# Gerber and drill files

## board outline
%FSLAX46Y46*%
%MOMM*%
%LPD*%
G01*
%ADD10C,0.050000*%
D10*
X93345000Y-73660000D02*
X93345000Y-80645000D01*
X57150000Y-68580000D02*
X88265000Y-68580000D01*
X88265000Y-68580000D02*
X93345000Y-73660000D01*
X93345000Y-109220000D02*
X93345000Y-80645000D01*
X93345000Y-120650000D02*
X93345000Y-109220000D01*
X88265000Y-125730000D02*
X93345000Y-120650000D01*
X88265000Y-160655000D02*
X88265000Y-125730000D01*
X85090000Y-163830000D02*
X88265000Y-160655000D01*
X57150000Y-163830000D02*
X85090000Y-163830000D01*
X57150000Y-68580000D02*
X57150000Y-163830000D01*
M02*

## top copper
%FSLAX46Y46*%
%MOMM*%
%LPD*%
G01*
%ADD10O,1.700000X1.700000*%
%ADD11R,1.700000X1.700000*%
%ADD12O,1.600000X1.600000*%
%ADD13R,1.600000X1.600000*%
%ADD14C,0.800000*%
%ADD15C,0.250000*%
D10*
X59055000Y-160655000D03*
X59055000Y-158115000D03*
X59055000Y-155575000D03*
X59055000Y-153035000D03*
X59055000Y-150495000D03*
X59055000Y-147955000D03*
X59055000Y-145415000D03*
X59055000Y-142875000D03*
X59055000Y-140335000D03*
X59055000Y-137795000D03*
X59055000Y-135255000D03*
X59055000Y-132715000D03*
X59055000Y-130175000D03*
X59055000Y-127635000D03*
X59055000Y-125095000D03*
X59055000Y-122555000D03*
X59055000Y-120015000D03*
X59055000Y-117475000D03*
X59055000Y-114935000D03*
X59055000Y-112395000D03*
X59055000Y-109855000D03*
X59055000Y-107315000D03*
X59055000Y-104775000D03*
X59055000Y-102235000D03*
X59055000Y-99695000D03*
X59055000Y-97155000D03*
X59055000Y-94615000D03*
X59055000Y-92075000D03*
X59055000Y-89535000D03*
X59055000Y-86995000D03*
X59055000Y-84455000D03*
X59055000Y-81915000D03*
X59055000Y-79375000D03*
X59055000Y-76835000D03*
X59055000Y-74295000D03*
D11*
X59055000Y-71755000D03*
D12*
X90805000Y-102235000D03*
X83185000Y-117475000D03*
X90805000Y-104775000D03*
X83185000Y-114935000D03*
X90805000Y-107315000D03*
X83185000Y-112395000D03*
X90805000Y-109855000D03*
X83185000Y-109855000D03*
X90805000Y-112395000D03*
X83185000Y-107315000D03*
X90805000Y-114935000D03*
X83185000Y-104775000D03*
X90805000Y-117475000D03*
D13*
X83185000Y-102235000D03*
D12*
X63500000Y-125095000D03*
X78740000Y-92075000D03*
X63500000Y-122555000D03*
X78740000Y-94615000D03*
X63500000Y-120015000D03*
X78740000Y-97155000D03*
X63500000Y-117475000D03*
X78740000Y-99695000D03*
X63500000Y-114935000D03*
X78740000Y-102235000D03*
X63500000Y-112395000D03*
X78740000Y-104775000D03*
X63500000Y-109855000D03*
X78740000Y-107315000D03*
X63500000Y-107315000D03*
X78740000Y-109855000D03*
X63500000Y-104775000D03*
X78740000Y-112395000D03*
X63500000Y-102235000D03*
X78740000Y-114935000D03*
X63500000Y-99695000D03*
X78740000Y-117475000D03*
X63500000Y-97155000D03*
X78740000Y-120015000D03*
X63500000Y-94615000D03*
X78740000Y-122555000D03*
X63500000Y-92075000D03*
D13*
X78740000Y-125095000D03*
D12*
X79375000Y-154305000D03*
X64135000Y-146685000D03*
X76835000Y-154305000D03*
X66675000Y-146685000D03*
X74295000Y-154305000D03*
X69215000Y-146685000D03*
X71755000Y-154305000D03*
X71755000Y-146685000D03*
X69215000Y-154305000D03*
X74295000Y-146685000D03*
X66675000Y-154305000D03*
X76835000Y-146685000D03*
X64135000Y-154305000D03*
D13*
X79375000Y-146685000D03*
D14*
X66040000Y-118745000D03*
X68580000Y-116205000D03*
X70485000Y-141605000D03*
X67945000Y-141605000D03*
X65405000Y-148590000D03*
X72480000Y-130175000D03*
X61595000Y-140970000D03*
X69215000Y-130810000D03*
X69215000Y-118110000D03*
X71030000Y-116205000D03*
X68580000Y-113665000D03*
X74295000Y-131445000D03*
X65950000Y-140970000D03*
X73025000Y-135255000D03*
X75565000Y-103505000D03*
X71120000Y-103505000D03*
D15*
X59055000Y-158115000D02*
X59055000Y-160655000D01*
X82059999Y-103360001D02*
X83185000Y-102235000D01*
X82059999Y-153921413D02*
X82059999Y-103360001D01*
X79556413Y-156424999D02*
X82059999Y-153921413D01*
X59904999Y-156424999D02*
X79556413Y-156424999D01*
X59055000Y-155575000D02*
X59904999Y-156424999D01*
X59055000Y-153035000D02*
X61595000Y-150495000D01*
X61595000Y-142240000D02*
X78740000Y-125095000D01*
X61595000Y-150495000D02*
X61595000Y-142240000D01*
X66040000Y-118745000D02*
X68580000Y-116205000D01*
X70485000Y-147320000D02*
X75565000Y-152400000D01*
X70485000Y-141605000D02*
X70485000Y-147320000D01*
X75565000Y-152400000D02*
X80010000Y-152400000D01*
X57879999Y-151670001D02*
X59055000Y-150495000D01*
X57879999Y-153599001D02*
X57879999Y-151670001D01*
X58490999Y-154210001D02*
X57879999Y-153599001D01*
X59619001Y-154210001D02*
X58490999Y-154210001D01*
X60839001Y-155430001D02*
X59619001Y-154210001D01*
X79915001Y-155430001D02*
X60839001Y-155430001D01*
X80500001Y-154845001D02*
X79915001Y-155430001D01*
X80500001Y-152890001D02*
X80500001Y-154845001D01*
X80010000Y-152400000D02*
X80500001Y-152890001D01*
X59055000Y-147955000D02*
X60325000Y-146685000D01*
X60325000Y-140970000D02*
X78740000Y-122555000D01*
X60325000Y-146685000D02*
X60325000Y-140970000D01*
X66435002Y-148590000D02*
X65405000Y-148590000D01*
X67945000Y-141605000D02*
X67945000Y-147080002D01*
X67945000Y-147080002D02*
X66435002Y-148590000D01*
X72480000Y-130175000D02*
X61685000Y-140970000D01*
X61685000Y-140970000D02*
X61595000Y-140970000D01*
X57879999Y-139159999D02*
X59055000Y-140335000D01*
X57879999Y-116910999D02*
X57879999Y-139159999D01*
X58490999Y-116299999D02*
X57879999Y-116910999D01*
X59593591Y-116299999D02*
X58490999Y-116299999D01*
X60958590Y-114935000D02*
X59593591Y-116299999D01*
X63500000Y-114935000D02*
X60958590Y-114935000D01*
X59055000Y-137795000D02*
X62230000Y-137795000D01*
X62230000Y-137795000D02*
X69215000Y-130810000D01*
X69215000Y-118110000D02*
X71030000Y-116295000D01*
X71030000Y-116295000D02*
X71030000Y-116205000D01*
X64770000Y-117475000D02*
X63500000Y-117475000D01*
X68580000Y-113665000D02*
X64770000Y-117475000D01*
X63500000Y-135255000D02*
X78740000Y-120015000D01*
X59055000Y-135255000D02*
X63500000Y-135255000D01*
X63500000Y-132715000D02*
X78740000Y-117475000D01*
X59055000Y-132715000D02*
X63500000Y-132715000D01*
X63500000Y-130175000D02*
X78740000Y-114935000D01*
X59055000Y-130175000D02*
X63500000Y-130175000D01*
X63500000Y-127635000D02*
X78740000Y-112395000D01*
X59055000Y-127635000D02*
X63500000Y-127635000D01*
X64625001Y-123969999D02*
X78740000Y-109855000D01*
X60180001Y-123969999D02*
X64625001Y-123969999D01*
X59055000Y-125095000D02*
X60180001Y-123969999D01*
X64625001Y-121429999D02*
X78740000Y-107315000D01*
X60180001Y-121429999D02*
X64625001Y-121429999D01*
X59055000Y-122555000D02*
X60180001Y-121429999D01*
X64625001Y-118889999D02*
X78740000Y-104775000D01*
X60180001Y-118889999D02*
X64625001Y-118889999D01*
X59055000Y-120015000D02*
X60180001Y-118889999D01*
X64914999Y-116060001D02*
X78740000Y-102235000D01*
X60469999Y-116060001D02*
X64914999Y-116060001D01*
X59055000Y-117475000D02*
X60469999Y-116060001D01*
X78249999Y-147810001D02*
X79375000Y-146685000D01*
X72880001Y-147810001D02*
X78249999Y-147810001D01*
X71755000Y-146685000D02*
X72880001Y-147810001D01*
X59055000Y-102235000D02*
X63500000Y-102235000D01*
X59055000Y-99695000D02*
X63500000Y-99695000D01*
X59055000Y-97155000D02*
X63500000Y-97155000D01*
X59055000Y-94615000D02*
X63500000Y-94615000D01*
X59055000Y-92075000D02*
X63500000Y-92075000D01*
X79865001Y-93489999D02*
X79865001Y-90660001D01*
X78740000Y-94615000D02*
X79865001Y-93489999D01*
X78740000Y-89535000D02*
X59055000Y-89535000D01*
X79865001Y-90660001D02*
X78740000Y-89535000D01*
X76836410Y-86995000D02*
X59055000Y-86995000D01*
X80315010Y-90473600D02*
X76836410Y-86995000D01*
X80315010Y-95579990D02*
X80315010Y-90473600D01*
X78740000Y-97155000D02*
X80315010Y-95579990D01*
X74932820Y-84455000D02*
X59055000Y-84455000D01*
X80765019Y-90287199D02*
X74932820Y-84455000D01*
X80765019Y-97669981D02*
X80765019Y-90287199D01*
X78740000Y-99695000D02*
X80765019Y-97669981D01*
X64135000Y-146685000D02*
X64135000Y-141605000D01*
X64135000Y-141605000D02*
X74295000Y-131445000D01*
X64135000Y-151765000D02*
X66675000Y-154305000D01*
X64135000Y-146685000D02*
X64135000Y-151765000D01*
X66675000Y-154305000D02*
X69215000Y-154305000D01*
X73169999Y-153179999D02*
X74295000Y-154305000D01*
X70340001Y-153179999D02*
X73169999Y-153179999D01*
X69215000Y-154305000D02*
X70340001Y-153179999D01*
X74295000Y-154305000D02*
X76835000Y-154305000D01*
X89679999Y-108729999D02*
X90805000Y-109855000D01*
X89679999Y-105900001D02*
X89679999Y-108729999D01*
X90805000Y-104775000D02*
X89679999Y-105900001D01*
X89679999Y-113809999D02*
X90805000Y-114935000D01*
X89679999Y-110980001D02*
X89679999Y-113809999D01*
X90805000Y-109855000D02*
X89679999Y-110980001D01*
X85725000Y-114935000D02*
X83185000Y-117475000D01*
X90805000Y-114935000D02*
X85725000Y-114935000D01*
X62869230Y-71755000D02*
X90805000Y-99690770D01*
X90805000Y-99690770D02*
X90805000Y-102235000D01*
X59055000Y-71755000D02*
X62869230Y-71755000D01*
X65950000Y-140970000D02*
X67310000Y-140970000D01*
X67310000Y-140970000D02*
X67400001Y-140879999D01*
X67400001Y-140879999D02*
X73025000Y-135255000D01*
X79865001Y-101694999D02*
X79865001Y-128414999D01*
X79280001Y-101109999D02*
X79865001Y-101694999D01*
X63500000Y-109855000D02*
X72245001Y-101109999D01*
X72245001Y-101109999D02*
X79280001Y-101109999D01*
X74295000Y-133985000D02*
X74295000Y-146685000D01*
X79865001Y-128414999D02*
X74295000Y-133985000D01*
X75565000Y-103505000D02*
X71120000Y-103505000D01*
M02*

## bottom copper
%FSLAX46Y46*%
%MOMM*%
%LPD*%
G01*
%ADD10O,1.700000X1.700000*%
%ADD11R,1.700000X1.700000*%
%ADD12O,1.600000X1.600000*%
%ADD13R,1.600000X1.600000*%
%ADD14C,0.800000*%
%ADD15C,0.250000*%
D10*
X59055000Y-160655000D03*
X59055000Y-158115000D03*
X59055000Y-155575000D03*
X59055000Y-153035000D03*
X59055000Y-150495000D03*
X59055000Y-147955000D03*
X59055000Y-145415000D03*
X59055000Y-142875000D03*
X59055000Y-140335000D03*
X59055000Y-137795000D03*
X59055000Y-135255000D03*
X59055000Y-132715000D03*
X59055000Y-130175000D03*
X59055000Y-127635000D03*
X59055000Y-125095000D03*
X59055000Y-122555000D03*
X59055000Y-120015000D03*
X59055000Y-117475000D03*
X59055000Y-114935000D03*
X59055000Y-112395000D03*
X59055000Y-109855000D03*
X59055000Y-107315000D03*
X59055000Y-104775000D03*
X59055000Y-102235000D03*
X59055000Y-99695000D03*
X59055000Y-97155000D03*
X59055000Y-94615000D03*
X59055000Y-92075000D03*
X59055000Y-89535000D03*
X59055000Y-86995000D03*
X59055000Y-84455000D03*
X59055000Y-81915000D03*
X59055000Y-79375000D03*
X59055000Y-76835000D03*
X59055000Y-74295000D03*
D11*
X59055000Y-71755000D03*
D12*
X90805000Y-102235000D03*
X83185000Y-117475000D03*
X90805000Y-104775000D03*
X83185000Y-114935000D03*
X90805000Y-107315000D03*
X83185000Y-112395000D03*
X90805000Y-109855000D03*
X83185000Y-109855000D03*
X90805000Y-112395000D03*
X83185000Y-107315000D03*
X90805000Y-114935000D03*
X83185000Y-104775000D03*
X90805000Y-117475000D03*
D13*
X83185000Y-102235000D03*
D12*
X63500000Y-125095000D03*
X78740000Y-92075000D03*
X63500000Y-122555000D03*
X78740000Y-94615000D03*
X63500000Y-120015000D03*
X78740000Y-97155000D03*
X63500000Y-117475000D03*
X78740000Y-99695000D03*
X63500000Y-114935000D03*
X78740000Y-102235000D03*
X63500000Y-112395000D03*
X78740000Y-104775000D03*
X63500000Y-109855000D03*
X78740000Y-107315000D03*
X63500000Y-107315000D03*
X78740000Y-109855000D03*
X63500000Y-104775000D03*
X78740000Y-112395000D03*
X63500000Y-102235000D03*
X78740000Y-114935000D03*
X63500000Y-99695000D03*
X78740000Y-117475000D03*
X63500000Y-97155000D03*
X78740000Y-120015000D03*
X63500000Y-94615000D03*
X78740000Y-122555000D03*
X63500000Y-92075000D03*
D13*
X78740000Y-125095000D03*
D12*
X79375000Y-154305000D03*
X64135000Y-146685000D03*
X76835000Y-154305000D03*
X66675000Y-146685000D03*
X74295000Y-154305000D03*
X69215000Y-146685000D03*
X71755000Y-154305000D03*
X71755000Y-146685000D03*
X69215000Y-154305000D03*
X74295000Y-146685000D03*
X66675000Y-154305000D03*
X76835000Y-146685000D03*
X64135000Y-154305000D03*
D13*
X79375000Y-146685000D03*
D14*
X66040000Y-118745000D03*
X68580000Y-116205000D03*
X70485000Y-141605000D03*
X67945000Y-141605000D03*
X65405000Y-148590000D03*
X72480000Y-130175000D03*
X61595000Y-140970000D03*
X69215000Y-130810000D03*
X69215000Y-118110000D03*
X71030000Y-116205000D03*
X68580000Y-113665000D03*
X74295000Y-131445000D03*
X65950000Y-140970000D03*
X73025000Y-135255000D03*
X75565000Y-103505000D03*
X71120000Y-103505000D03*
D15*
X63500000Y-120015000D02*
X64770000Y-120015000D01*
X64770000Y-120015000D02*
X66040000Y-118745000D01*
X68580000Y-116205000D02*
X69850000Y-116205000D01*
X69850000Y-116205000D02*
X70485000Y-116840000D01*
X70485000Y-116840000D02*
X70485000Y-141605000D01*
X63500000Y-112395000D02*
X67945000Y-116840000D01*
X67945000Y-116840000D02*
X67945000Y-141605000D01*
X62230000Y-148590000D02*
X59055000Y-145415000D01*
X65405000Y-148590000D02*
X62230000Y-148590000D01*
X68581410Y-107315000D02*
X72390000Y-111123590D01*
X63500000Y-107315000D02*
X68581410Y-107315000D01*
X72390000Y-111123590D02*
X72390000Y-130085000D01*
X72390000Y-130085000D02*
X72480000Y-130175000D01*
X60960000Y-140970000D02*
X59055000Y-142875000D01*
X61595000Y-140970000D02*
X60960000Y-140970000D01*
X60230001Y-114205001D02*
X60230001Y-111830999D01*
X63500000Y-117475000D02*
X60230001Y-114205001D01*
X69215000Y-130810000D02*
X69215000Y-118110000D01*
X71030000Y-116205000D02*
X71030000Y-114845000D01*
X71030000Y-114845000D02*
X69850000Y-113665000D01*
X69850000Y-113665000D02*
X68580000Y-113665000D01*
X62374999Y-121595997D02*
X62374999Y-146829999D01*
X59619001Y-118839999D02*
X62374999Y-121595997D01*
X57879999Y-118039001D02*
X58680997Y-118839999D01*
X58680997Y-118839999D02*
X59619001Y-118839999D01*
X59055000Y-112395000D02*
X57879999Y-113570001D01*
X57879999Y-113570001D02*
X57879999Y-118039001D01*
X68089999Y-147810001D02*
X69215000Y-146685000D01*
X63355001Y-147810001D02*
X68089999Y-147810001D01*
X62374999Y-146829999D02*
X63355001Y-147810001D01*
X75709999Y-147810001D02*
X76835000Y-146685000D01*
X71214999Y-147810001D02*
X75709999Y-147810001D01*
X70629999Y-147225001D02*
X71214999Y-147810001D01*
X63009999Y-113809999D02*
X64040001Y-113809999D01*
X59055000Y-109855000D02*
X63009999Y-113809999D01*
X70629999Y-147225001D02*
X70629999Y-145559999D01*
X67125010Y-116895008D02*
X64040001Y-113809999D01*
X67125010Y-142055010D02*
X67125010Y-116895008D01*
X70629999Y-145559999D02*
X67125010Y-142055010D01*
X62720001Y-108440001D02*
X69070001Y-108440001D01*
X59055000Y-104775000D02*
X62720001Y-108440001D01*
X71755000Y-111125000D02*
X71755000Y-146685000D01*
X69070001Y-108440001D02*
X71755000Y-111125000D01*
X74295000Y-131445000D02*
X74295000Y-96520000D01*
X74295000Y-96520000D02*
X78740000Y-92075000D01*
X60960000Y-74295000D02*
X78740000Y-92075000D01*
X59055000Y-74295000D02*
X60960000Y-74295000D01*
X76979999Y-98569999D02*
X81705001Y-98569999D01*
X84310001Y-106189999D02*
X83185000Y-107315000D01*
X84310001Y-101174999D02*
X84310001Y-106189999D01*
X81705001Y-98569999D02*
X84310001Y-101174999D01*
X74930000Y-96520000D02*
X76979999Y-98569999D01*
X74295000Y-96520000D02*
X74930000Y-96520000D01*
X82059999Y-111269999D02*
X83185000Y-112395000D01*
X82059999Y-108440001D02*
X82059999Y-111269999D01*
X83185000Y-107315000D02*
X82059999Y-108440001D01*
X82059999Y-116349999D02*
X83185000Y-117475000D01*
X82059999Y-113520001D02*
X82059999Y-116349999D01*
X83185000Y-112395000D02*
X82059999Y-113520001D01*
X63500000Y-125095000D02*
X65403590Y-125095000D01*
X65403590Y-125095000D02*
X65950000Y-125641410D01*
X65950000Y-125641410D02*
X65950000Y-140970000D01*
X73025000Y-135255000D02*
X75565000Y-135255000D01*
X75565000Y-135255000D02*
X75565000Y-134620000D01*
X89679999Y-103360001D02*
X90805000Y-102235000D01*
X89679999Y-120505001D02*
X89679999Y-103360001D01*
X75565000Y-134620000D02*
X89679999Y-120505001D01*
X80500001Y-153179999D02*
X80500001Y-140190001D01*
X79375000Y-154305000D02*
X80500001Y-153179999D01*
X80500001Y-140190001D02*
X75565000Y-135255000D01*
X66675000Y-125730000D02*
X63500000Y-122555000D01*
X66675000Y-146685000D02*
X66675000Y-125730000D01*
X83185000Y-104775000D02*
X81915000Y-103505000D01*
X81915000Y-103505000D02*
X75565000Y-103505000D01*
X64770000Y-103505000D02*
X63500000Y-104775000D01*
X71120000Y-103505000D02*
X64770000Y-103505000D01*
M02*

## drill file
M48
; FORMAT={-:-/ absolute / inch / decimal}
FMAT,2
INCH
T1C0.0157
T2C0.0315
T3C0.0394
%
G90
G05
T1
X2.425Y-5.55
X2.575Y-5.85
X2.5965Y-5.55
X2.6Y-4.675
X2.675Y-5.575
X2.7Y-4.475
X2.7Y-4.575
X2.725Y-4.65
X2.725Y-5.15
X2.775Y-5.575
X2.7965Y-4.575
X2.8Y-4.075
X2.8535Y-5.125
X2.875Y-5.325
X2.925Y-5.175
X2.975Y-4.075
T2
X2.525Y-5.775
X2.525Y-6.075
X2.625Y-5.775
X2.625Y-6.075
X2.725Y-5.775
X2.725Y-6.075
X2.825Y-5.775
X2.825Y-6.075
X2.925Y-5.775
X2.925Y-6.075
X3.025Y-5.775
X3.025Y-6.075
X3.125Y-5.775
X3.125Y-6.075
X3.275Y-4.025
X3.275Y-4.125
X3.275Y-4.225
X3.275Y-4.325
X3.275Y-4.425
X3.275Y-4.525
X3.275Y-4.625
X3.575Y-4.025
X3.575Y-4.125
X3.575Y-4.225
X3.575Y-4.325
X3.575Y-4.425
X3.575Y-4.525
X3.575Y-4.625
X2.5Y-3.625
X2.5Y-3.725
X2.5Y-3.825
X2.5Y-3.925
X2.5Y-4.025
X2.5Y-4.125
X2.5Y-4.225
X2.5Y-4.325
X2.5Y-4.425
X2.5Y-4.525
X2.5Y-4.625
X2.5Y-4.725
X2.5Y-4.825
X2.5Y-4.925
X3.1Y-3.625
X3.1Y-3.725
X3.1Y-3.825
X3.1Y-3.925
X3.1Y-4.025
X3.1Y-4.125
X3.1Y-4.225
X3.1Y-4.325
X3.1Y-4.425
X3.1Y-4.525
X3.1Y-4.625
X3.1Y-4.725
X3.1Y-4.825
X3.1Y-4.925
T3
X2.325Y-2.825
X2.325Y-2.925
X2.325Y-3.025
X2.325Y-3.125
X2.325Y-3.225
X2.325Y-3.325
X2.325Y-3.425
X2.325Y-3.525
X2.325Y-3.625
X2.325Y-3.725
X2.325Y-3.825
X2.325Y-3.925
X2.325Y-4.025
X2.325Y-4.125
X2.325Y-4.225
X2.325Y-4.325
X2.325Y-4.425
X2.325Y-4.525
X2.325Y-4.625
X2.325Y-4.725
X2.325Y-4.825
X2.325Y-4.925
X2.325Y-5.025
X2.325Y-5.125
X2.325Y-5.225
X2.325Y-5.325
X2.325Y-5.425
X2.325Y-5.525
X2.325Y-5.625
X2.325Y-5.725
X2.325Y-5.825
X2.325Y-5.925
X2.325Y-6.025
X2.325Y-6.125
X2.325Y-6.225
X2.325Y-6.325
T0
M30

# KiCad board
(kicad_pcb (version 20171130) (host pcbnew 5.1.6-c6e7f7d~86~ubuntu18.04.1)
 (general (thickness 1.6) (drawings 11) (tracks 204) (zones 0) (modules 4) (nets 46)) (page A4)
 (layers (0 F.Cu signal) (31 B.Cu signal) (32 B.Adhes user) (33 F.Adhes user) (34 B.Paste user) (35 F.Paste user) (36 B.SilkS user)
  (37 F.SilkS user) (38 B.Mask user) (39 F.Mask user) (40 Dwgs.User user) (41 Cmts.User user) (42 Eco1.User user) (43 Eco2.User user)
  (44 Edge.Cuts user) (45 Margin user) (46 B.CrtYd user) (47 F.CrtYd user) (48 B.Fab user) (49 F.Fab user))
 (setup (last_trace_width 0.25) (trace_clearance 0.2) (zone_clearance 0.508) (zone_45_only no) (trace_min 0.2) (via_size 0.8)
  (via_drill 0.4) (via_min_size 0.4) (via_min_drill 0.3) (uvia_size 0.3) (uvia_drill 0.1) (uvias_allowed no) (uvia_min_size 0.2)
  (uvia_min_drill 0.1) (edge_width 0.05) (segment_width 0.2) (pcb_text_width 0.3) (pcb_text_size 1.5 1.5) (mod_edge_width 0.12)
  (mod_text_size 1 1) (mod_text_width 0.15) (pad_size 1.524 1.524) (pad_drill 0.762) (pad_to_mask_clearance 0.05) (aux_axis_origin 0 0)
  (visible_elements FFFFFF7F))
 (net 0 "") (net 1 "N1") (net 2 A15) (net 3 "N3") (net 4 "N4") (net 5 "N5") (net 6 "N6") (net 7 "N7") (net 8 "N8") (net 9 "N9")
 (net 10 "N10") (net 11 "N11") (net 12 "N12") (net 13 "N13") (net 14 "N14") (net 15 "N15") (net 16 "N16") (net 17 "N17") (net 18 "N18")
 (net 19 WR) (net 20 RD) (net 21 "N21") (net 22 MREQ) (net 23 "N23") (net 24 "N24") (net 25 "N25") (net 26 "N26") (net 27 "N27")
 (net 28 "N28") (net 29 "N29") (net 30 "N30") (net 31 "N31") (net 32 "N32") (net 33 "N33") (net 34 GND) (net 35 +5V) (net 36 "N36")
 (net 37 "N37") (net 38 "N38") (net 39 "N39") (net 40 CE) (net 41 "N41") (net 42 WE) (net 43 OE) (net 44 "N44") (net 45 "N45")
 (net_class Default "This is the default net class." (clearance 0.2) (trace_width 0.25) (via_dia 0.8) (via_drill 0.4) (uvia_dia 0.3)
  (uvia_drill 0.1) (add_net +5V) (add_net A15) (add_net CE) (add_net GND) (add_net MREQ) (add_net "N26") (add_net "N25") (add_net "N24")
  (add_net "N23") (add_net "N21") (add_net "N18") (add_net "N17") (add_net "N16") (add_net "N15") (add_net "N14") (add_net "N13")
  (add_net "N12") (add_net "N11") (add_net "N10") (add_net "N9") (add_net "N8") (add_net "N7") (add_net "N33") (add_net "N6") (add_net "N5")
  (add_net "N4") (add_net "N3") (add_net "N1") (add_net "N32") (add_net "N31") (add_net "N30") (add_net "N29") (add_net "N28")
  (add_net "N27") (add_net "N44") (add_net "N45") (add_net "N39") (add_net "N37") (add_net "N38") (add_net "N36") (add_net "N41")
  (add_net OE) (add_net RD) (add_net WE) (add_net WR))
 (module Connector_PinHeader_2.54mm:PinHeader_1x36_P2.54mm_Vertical (layer F.Cu) (at 59.055 71.755)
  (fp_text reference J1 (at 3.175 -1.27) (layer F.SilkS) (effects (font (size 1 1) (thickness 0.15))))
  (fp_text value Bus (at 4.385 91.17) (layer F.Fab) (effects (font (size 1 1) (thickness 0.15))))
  (pad 36 thru_hole oval (at 0 88.9) (size 1.7 1.7) (drill 1) (layers *.Cu *.Mask) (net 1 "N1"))
  (pad 35 thru_hole oval (at 0 86.36) (size 1.7 1.7) (drill 1) (layers *.Cu *.Mask) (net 1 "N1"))
  (pad 34 thru_hole oval (at 0 83.82) (size 1.7 1.7) (drill 1) (layers *.Cu *.Mask) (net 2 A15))
  (pad 33 thru_hole oval (at 0 81.28) (size 1.7 1.7) (drill 1) (layers *.Cu *.Mask) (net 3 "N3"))
  (pad 32 thru_hole oval (at 0 78.74) (size 1.7 1.7) (drill 1) (layers *.Cu *.Mask) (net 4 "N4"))
  (pad 31 thru_hole oval (at 0 76.2) (size 1.7 1.7) (drill 1) (layers *.Cu *.Mask) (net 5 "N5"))
  (pad 30 thru_hole oval (at 0 73.66) (size 1.7 1.7) (drill 1) (layers *.Cu *.Mask) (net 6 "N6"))
  (pad 29 thru_hole oval (at 0 71.12) (size 1.7 1.7) (drill 1) (layers *.Cu *.Mask) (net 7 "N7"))
  (pad 28 thru_hole oval (at 0 68.58) (size 1.7 1.7) (drill 1) (layers *.Cu *.Mask) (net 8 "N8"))
  (pad 27 thru_hole oval (at 0 66.04) (size 1.7 1.7) (drill 1) (layers *.Cu *.Mask) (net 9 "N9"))
  (pad 26 thru_hole oval (at 0 63.5) (size 1.7 1.7) (drill 1) (layers *.Cu *.Mask) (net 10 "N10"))
  (pad 25 thru_hole oval (at 0 60.96) (size 1.7 1.7) (drill 1) (layers *.Cu *.Mask) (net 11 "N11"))
  (pad 24 thru_hole oval (at 0 58.42) (size 1.7 1.7) (drill 1) (layers *.Cu *.Mask) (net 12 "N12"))
  (pad 23 thru_hole oval (at 0 55.88) (size 1.7 1.7) (drill 1) (layers *.Cu *.Mask) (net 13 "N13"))
  (pad 22 thru_hole oval (at 0 53.34) (size 1.7 1.7) (drill 1) (layers *.Cu *.Mask) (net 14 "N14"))
  (pad 21 thru_hole oval (at 0 50.8) (size 1.7 1.7) (drill 1) (layers *.Cu *.Mask) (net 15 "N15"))
  (pad 20 thru_hole oval (at 0 48.26) (size 1.7 1.7) (drill 1) (layers *.Cu *.Mask) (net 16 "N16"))
  (pad 19 thru_hole oval (at 0 45.72) (size 1.7 1.7) (drill 1) (layers *.Cu *.Mask) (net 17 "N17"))
  (pad 18 thru_hole oval (at 0 43.18) (size 1.7 1.7) (drill 1) (layers *.Cu *.Mask) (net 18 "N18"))
  (pad 17 thru_hole oval (at 0 40.64) (size 1.7 1.7) (drill 1) (layers *.Cu *.Mask) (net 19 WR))
  (pad 16 thru_hole oval (at 0 38.1) (size 1.7 1.7) (drill 1) (layers *.Cu *.Mask) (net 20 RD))
  (pad 15 thru_hole oval (at 0 35.56) (size 1.7 1.7) (drill 1) (layers *.Cu *.Mask) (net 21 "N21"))
  (pad 14 thru_hole oval (at 0 33.02) (size 1.7 1.7) (drill 1) (layers *.Cu *.Mask) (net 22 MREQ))
  (pad 13 thru_hole oval (at 0 30.48) (size 1.7 1.7) (drill 1) (layers *.Cu *.Mask) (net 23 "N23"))
  (pad 12 thru_hole oval (at 0 27.94) (size 1.7 1.7) (drill 1) (layers *.Cu *.Mask) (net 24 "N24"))
  (pad 11 thru_hole oval (at 0 25.4) (size 1.7 1.7) (drill 1) (layers *.Cu *.Mask) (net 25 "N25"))
  (pad 10 thru_hole oval (at 0 22.86) (size 1.7 1.7) (drill 1) (layers *.Cu *.Mask) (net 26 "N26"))
  (pad 9 thru_hole oval (at 0 20.32) (size 1.7 1.7) (drill 1) (layers *.Cu *.Mask) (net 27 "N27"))
  (pad 8 thru_hole oval (at 0 17.78) (size 1.7 1.7) (drill 1) (layers *.Cu *.Mask) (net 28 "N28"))
  (pad 7 thru_hole oval (at 0 15.24) (size 1.7 1.7) (drill 1) (layers *.Cu *.Mask) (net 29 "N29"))
  (pad 6 thru_hole oval (at 0 12.7) (size 1.7 1.7) (drill 1) (layers *.Cu *.Mask) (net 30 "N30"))
  (pad 5 thru_hole oval (at 0 10.16) (size 1.7 1.7) (drill 1) (layers *.Cu *.Mask) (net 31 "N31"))
  (pad 4 thru_hole oval (at 0 7.62) (size 1.7 1.7) (drill 1) (layers *.Cu *.Mask) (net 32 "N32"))
  (pad 3 thru_hole oval (at 0 5.08) (size 1.7 1.7) (drill 1) (layers *.Cu *.Mask) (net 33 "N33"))
  (pad 2 thru_hole oval (at 0 2.54) (size 1.7 1.7) (drill 1) (layers *.Cu *.Mask) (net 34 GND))
  (pad 1 thru_hole rect (at 0 0) (size 1.7 1.7) (drill 1) (layers *.Cu *.Mask) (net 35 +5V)))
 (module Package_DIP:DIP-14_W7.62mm (layer F.Cu) (at 83.185 102.235)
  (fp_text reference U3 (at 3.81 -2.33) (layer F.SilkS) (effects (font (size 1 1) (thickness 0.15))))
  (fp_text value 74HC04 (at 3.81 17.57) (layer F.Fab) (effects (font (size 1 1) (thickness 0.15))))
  (pad 14 thru_hole oval (at 7.62 0) (size 1.6 1.6) (drill 0.8) (layers *.Cu *.Mask) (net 35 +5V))
  (pad 7 thru_hole oval (at 0 15.24) (size 1.6 1.6) (drill 0.8) (layers *.Cu *.Mask) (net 34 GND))
  (pad 13 thru_hole oval (at 7.62 2.54) (size 1.6 1.6) (drill 0.8) (layers *.Cu *.Mask) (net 34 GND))
  (pad 6 thru_hole oval (at 0 12.7) (size 1.6 1.6) (drill 0.8) (layers *.Cu *.Mask) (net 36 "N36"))
  (pad 12 thru_hole oval (at 7.62 5.08) (size 1.6 1.6) (drill 0.8) (layers *.Cu *.Mask) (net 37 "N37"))
  (pad 5 thru_hole oval (at 0 10.16) (size 1.6 1.6) (drill 0.8) (layers *.Cu *.Mask) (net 34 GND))
  (pad 11 thru_hole oval (at 7.62 7.62) (size 1.6 1.6) (drill 0.8) (layers *.Cu *.Mask) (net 34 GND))
  (pad 4 thru_hole oval (at 0 7.62) (size 1.6 1.6) (drill 0.8) (layers *.Cu *.Mask) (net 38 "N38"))
  (pad 10 thru_hole oval (at 7.62 10.16) (size 1.6 1.6) (drill 0.8) (layers *.Cu *.Mask) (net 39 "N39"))
  (pad 3 thru_hole oval (at 0 5.08) (size 1.6 1.6) (drill 0.8) (layers *.Cu *.Mask) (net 34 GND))
  (pad 9 thru_hole oval (at 7.62 12.7) (size 1.6 1.6) (drill 0.8) (layers *.Cu *.Mask) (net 34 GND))
  (pad 2 thru_hole oval (at 0 2.54) (size 1.6 1.6) (drill 0.8) (layers *.Cu *.Mask) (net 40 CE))
  (pad 8 thru_hole oval (at 7.62 15.24) (size 1.6 1.6) (drill 0.8) (layers *.Cu *.Mask) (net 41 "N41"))
  (pad 1 thru_hole rect (at 0 0) (size 1.6 1.6) (drill 0.8) (layers *.Cu *.Mask) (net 2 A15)))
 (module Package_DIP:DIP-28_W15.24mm (layer F.Cu) (at 78.74 125.095 180)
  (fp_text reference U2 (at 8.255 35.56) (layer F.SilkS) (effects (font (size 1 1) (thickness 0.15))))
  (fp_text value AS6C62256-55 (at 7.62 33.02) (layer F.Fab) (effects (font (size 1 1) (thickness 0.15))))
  (pad 28 thru_hole oval (at 15.24 0 180) (size 1.6 1.6) (drill 0.8) (layers *.Cu *.Mask) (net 35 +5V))
  (pad 14 thru_hole oval (at 0 33.02 180) (size 1.6 1.6) (drill 0.8) (layers *.Cu *.Mask) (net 34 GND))
  (pad 27 thru_hole oval (at 15.24 2.54 180) (size 1.6 1.6) (drill 0.8) (layers *.Cu *.Mask) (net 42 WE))
  (pad 13 thru_hole oval (at 0 30.48 180) (size 1.6 1.6) (drill 0.8) (layers *.Cu *.Mask) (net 28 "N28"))
  (pad 26 thru_hole oval (at 15.24 5.08 180) (size 1.6 1.6) (drill 0.8) (layers *.Cu *.Mask) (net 4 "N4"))
  (pad 12 thru_hole oval (at 0 27.94 180) (size 1.6 1.6) (drill 0.8) (layers *.Cu *.Mask) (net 29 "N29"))
  (pad 25 thru_hole oval (at 15.24 7.62 180) (size 1.6 1.6) (drill 0.8) (layers *.Cu *.Mask) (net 9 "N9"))
  (pad 11 thru_hole oval (at 0 25.4 180) (size 1.6 1.6) (drill 0.8) (layers *.Cu *.Mask) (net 30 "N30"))
  (pad 24 thru_hole oval (at 15.24 10.16 180) (size 1.6 1.6) (drill 0.8) (layers *.Cu *.Mask) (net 8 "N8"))
  (pad 10 thru_hole oval (at 0 22.86 180) (size 1.6 1.6) (drill 0.8) (layers *.Cu *.Mask) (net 17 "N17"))
  (pad 23 thru_hole oval (at 15.24 12.7 180) (size 1.6 1.6) (drill 0.8) (layers *.Cu *.Mask) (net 6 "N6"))
  (pad 9 thru_hole oval (at 0 20.32 180) (size 1.6 1.6) (drill 0.8) (layers *.Cu *.Mask) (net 16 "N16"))
  (pad 22 thru_hole oval (at 15.24 15.24 180) (size 1.6 1.6) (drill 0.8) (layers *.Cu *.Mask) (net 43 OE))
  (pad 8 thru_hole oval (at 0 17.78 180) (size 1.6 1.6) (drill 0.8) (layers *.Cu *.Mask) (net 15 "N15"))
  (pad 21 thru_hole oval (at 15.24 17.78 180) (size 1.6 1.6) (drill 0.8) (layers *.Cu *.Mask) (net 7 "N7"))
  (pad 7 thru_hole oval (at 0 15.24 180) (size 1.6 1.6) (drill 0.8) (layers *.Cu *.Mask) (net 14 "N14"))
  (pad 20 thru_hole oval (at 15.24 20.32 180) (size 1.6 1.6) (drill 0.8) (layers *.Cu *.Mask) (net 40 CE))
  (pad 6 thru_hole oval (at 0 12.7 180) (size 1.6 1.6) (drill 0.8) (layers *.Cu *.Mask) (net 13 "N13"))
  (pad 19 thru_hole oval (at 15.24 22.86 180) (size 1.6 1.6) (drill 0.8) (layers *.Cu *.Mask) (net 23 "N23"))
  (pad 5 thru_hole oval (at 0 10.16 180) (size 1.6 1.6) (drill 0.8) (layers *.Cu *.Mask) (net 12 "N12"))
  (pad 18 thru_hole oval (at 15.24 25.4 180) (size 1.6 1.6) (drill 0.8) (layers *.Cu *.Mask) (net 24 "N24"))
  (pad 4 thru_hole oval (at 0 7.62 180) (size 1.6 1.6) (drill 0.8) (layers *.Cu *.Mask) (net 11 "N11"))
  (pad 17 thru_hole oval (at 15.24 27.94 180) (size 1.6 1.6) (drill 0.8) (layers *.Cu *.Mask) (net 25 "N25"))
  (pad 3 thru_hole oval (at 0 5.08 180) (size 1.6 1.6) (drill 0.8) (layers *.Cu *.Mask) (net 10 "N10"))
  (pad 16 thru_hole oval (at 15.24 30.48 180) (size 1.6 1.6) (drill 0.8) (layers *.Cu *.Mask) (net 26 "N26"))
  (pad 2 thru_hole oval (at 0 2.54 180) (size 1.6 1.6) (drill 0.8) (layers *.Cu *.Mask) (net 5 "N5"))
  (pad 15 thru_hole oval (at 15.24 33.02 180) (size 1.6 1.6) (drill 0.8) (layers *.Cu *.Mask) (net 27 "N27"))
  (pad 1 thru_hole rect (at 0 0 180) (size 1.6 1.6) (drill 0.8) (layers *.Cu *.Mask) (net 3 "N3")))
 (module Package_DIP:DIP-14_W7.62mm (layer F.Cu) (at 79.375 146.685 270)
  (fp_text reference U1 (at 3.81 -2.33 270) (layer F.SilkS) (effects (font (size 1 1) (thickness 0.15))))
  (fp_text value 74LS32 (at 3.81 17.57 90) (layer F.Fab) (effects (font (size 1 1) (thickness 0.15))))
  (pad 14 thru_hole oval (at 7.62 0 270) (size 1.6 1.6) (drill 0.8) (layers *.Cu *.Mask) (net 35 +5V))
  (pad 7 thru_hole oval (at 0 15.24 270) (size 1.6 1.6) (drill 0.8) (layers *.Cu *.Mask) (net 34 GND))
  (pad 13 thru_hole oval (at 7.62 2.54 270) (size 1.6 1.6) (drill 0.8) (layers *.Cu *.Mask) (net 34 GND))
  (pad 6 thru_hole oval (at 0 12.7 270) (size 1.6 1.6) (drill 0.8) (layers *.Cu *.Mask) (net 42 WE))
  (pad 12 thru_hole oval (at 7.62 5.08 270) (size 1.6 1.6) (drill 0.8) (layers *.Cu *.Mask) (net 34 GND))
  (pad 5 thru_hole oval (at 0 10.16 270) (size 1.6 1.6) (drill 0.8) (layers *.Cu *.Mask) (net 19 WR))
  (pad 11 thru_hole oval (at 7.62 7.62 270) (size 1.6 1.6) (drill 0.8) (layers *.Cu *.Mask) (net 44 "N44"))
  (pad 4 thru_hole oval (at 0 7.62 270) (size 1.6 1.6) (drill 0.8) (layers *.Cu *.Mask) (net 22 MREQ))
  (pad 10 thru_hole oval (at 7.62 10.16 270) (size 1.6 1.6) (drill 0.8) (layers *.Cu *.Mask) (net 34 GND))
  (pad 3 thru_hole oval (at 0 5.08 270) (size 1.6 1.6) (drill 0.8) (layers *.Cu *.Mask) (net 43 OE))
  (pad 9 thru_hole oval (at 7.62 12.7 270) (size 1.6 1.6) (drill 0.8) (layers *.Cu *.Mask) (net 34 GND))
  (pad 2 thru_hole oval (at 0 2.54 270) (size 1.6 1.6) (drill 0.8) (layers *.Cu *.Mask) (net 20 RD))
  (pad 8 thru_hole oval (at 7.62 15.24 270) (size 1.6 1.6) (drill 0.8) (layers *.Cu *.Mask) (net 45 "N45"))
  (pad 1 thru_hole rect (at 0 0 270) (size 1.6 1.6) (drill 0.8) (layers *.Cu *.Mask) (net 22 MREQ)))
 (gr_line (start 93.345 73.66) (end 93.345 80.645) (layer Edge.Cuts) (width 0.05))
 (gr_line (start 57.15 68.58) (end 88.265 68.58) (layer Edge.Cuts) (width 0.05))
 (gr_line (start 88.265 68.58) (end 93.345 73.66) (layer Edge.Cuts) (width 0.05))
 (gr_line (start 93.345 109.22) (end 93.345 80.645) (layer Edge.Cuts) (width 0.05))
 (gr_line (start 93.345 120.65) (end 93.345 109.22) (layer Edge.Cuts) (width 0.05))
 (gr_line (start 88.265 125.73) (end 93.345 120.65) (layer Edge.Cuts) (width 0.05))
 (gr_line (start 88.265 160.655) (end 88.265 125.73) (layer Edge.Cuts) (width 0.05))
 (gr_line (start 85.09 163.83) (end 88.265 160.655) (layer Edge.Cuts) (width 0.05))
 (gr_line (start 57.15 163.83) (end 85.09 163.83) (layer Edge.Cuts) (width 0.05))
 (gr_line (start 57.15 68.58) (end 57.15 163.83) (layer Edge.Cuts) (width 0.05))
 (segment (start 59.055 158.115) (end 59.055 160.655) (width 0.25) (layer F.Cu) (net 1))
 (segment (start 82.059999 103.360001) (end 83.185 102.235) (width 0.25) (layer F.Cu) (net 2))
 (segment (start 82.059999 153.921413) (end 82.059999 103.360001) (width 0.25) (layer F.Cu) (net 2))
 (segment (start 79.556413 156.424999) (end 82.059999 153.921413) (width 0.25) (layer F.Cu) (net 2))
 (segment (start 59.904999 156.424999) (end 79.556413 156.424999) (width 0.25) (layer F.Cu) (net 2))
 (segment (start 59.055 155.575) (end 59.904999 156.424999) (width 0.25) (layer F.Cu) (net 2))
 (segment (start 59.055 153.035) (end 61.595 150.495) (width 0.25) (layer F.Cu) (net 3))
 (segment (start 61.595 142.24) (end 78.74 125.095) (width 0.25) (layer F.Cu) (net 3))
 (segment (start 61.595 150.495) (end 61.595 142.24) (width 0.25) (layer F.Cu) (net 3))
 (via (at 66.04 118.745) (size 0.8) (drill 0.4) (layers F.Cu B.Cu) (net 4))
 (segment (start 63.5 120.015) (end 64.77 120.015) (width 0.25) (layer B.Cu) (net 4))
 (segment (start 64.77 120.015) (end 66.04 118.745) (width 0.25) (layer B.Cu) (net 4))
 (via (at 68.58 116.205) (size 0.8) (drill 0.4) (layers F.Cu B.Cu) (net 4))
 (segment (start 66.04 118.745) (end 68.58 116.205) (width 0.25) (layer F.Cu) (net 4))
 (segment (start 68.58 116.205) (end 69.85 116.205) (width 0.25) (layer B.Cu) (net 4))
 (segment (start 69.85 116.205) (end 70.485 116.84) (width 0.25) (layer B.Cu) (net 4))
 (via (at 70.485 141.605) (size 0.8) (drill 0.4) (layers F.Cu B.Cu) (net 4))
 (segment (start 70.485 116.84) (end 70.485 141.605) (width 0.25) (layer B.Cu) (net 4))
 (segment (start 70.485 147.32) (end 75.565 152.4) (width 0.25) (layer F.Cu) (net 4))
 (segment (start 70.485 141.605) (end 70.485 147.32) (width 0.25) (layer F.Cu) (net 4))
 (segment (start 75.565 152.4) (end 80.01 152.4) (width 0.25) (layer F.Cu) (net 4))
 (segment (start 57.879999 151.670001) (end 59.055 150.495) (width 0.25) (layer F.Cu) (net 4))
 (segment (start 57.879999 153.599001) (end 57.879999 151.670001) (width 0.25) (layer F.Cu) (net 4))
 (segment (start 58.490999 154.210001) (end 57.879999 153.599001) (width 0.25) (layer F.Cu) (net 4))
 (segment (start 59.619001 154.210001) (end 58.490999 154.210001) (width 0.25) (layer F.Cu) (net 4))
 (segment (start 60.839001 155.430001) (end 59.619001 154.210001) (width 0.25) (layer F.Cu) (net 4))
 (segment (start 79.915001 155.430001) (end 60.839001 155.430001) (width 0.25) (layer F.Cu) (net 4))
 (segment (start 80.500001 154.845001) (end 79.915001 155.430001) (width 0.25) (layer F.Cu) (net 4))
 (segment (start 80.500001 152.890001) (end 80.500001 154.845001) (width 0.25) (layer F.Cu) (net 4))
 (segment (start 80.01 152.4) (end 80.500001 152.890001) (width 0.25) (layer F.Cu) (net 4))
 (segment (start 59.055 147.955) (end 60.325 146.685) (width 0.25) (layer F.Cu) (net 5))
 (segment (start 60.325 140.97) (end 78.74 122.555) (width 0.25) (layer F.Cu) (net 5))
 (segment (start 60.325 146.685) (end 60.325 140.97) (width 0.25) (layer F.Cu) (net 5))
 (segment (start 63.5 112.395) (end 67.945 116.84) (width 0.25) (layer B.Cu) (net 6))
 (via (at 67.945 141.605) (size 0.8) (drill 0.4) (layers F.Cu B.Cu) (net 6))
 (segment (start 67.945 116.84) (end 67.945 141.605) (width 0.25) (layer B.Cu) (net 6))
 (via (at 65.405 148.59) (size 0.8) (drill 0.4) (layers F.Cu B.Cu) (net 6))
 (segment (start 66.435002 148.59) (end 65.405 148.59) (width 0.25) (layer F.Cu) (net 6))
 (segment (start 67.945 141.605) (end 67.945 147.080002) (width 0.25) (layer F.Cu) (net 6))
 (segment (start 67.945 147.080002) (end 66.435002 148.59) (width 0.25) (layer F.Cu) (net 6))
 (segment (start 62.23 148.59) (end 59.055 145.415) (width 0.25) (layer B.Cu) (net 6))
 (segment (start 65.405 148.59) (end 62.23 148.59) (width 0.25) (layer B.Cu) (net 6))
 (segment (start 68.58141 107.315) (end 72.39 111.12359) (width 0.25) (layer B.Cu) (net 7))
 (segment (start 63.5 107.315) (end 68.58141 107.315) (width 0.25) (layer B.Cu) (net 7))
 (via (at 72.48 130.175) (size 0.8) (drill 0.4) (layers F.Cu B.Cu) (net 7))
 (segment (start 72.39 111.12359) (end 72.39 130.085) (width 0.25) (layer B.Cu) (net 7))
 (segment (start 72.39 130.085) (end 72.48 130.175) (width 0.25) (layer B.Cu) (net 7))
 (via (at 61.595 140.97) (size 0.8) (drill 0.4) (layers F.Cu B.Cu) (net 7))
 (segment (start 72.48 130.175) (end 61.685 140.97) (width 0.25) (layer F.Cu) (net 7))
 (segment (start 61.685 140.97) (end 61.595 140.97) (width 0.25) (layer F.Cu) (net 7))
 (segment (start 60.96 140.97) (end 59.055 142.875) (width 0.25) (layer B.Cu) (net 7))
 (segment (start 61.595 140.97) (end 60.96 140.97) (width 0.25) (layer B.Cu) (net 7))
 (segment (start 57.879999 139.159999) (end 59.055 140.335) (width 0.25) (layer F.Cu) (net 8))
 (segment (start 57.879999 116.910999) (end 57.879999 139.159999) (width 0.25) (layer F.Cu) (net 8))
 (segment (start 58.490999 116.299999) (end 57.879999 116.910999) (width 0.25) (layer F.Cu) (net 8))
 (segment (start 59.593591 116.299999) (end 58.490999 116.299999) (width 0.25) (layer F.Cu) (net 8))
 (segment (start 60.95859 114.935) (end 59.593591 116.299999) (width 0.25) (layer F.Cu) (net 8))
 (segment (start 63.5 114.935) (end 60.95859 114.935) (width 0.25) (layer F.Cu) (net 8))
 (segment (start 60.230001 114.205001) (end 60.230001 111.830999) (width 0.25) (layer B.Cu) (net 9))
 (segment (start 63.5 117.475) (end 60.230001 114.205001) (width 0.25) (layer B.Cu) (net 9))
 (segment (start 59.055 137.795) (end 62.23 137.795) (width 0.25) (layer F.Cu) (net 9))
 (via (at 69.215 130.81) (size 0.8) (drill 0.4) (layers F.Cu B.Cu) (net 9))
 (segment (start 62.23 137.795) (end 69.215 130.81) (width 0.25) (layer F.Cu) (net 9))
 (via (at 69.215 118.11) (size 0.8) (drill 0.4) (layers F.Cu B.Cu) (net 9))
 (segment (start 69.215 130.81) (end 69.215 118.11) (width 0.25) (layer B.Cu) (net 9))
 (via (at 71.03 116.205) (size 0.8) (drill 0.4) (layers F.Cu B.Cu) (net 9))
 (segment (start 69.215 118.11) (end 71.03 116.295) (width 0.25) (layer F.Cu) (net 9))
 (segment (start 71.03 116.295) (end 71.03 116.205) (width 0.25) (layer F.Cu) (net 9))
 (segment (start 71.03 116.205) (end 71.03 114.845) (width 0.25) (layer B.Cu) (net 9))
 (segment (start 71.03 114.845) (end 69.85 113.665) (width 0.25) (layer B.Cu) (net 9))
 (via (at 68.58 113.665) (size 0.8) (drill 0.4) (layers F.Cu B.Cu) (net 9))
 (segment (start 69.85 113.665) (end 68.58 113.665) (width 0.25) (layer B.Cu) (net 9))
 (segment (start 64.77 117.475) (end 63.5 117.475) (width 0.25) (layer F.Cu) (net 9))
 (segment (start 68.58 113.665) (end 64.77 117.475) (width 0.25) (layer F.Cu) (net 9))
 (segment (start 63.5 135.255) (end 78.74 120.015) (width 0.25) (layer F.Cu) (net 10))
 (segment (start 59.055 135.255) (end 63.5 135.255) (width 0.25) (layer F.Cu) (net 10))
 (segment (start 63.5 132.715) (end 78.74 117.475) (width 0.25) (layer F.Cu) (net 11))
 (segment (start 59.055 132.715) (end 63.5 132.715) (width 0.25) (layer F.Cu) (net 11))
 (segment (start 63.5 130.175) (end 78.74 114.935) (width 0.25) (layer F.Cu) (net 12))
 (segment (start 59.055 130.175) (end 63.5 130.175) (width 0.25) (layer F.Cu) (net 12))
 (segment (start 63.5 127.635) (end 78.74 112.395) (width 0.25) (layer F.Cu) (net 13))
 (segment (start 59.055 127.635) (end 63.5 127.635) (width 0.25) (layer F.Cu) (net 13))
 (segment (start 64.625001 123.969999) (end 78.74 109.855) (width 0.25) (layer F.Cu) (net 14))
 (segment (start 60.180001 123.969999) (end 64.625001 123.969999) (width 0.25) (layer F.Cu) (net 14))
 (segment (start 59.055 125.095) (end 60.180001 123.969999) (width 0.25) (layer F.Cu) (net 14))
 (segment (start 64.625001 121.429999) (end 78.74 107.315) (width 0.25) (layer F.Cu) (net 15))
 (segment (start 60.180001 121.429999) (end 64.625001 121.429999) (width 0.25) (layer F.Cu) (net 15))
 (segment (start 59.055 122.555) (end 60.180001 121.429999) (width 0.25) (layer F.Cu) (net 15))
 (segment (start 64.625001 118.889999) (end 78.74 104.775) (width 0.25) (layer F.Cu) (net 16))
 (segment (start 60.180001 118.889999) (end 64.625001 118.889999) (width 0.25) (layer F.Cu) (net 16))
 (segment (start 59.055 120.015) (end 60.180001 118.889999) (width 0.25) (layer F.Cu) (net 16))
 (segment (start 64.914999 116.060001) (end 78.74 102.235) (width 0.25) (layer F.Cu) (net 17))
 (segment (start 60.469999 116.060001) (end 64.914999 116.060001) (width 0.25) (layer F.Cu) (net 17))
 (segment (start 59.055 117.475) (end 60.469999 116.060001) (width 0.25) (layer F.Cu) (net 17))
 (segment (start 62.374999 121.595997) (end 62.374999 146.829999) (width 0.25) (layer B.Cu) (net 19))
 (segment (start 59.619001 118.839999) (end 62.374999 121.595997) (width 0.25) (layer B.Cu) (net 19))
 (segment (start 57.879999 118.039001) (end 58.680997 118.839999) (width 0.25) (layer B.Cu) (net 19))
 (segment (start 58.680997 118.839999) (end 59.619001 118.839999) (width 0.25) (layer B.Cu) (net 19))
 (segment (start 59.055 112.395) (end 57.879999 113.570001) (width 0.25) (layer B.Cu) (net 19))
 (segment (start 57.879999 113.570001) (end 57.879999 118.039001) (width 0.25) (layer B.Cu) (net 19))
 (segment (start 68.089999 147.810001) (end 69.215 146.685) (width 0.25) (layer B.Cu) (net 19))
 (segment (start 63.355001 147.810001) (end 68.089999 147.810001) (width 0.25) (layer B.Cu) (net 19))
 (segment (start 62.374999 146.829999) (end 63.355001 147.810001) (width 0.25) (layer B.Cu) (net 19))
 (segment (start 75.709999 147.810001) (end 76.835 146.685) (width 0.25) (layer B.Cu) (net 20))
 (segment (start 71.214999 147.810001) (end 75.709999 147.810001) (width 0.25) (layer B.Cu) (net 20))
 (segment (start 70.629999 147.225001) (end 71.214999 147.810001) (width 0.25) (layer B.Cu) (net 20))
 (segment (start 63.009999 113.809999) (end 64.040001 113.809999) (width 0.25) (layer B.Cu) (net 20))
 (segment (start 59.055 109.855) (end 63.009999 113.809999) (width 0.25) (layer B.Cu) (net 20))
 (segment (start 70.629999 147.225001) (end 70.629999 145.559999) (width 0.25) (layer B.Cu) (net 20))
 (segment (start 67.12501 116.895008) (end 64.040001 113.809999) (width 0.25) (layer B.Cu) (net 20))
 (segment (start 67.12501 142.05501) (end 67.12501 116.895008) (width 0.25) (layer B.Cu) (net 20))
 (segment (start 70.629999 145.559999) (end 67.12501 142.05501) (width 0.25) (layer B.Cu) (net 20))
 (segment (start 62.720001 108.440001) (end 69.070001 108.440001) (width 0.25) (layer B.Cu) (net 22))
 (segment (start 59.055 104.775) (end 62.720001 108.440001) (width 0.25) (layer B.Cu) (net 22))
 (segment (start 71.755 111.125) (end 71.755 146.685) (width 0.25) (layer B.Cu) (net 22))
 (segment (start 69.070001 108.440001) (end 71.755 111.125) (width 0.25) (layer B.Cu) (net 22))
 (segment (start 78.249999 147.810001) (end 79.375 146.685) (width 0.25) (layer F.Cu) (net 22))
 (segment (start 72.880001 147.810001) (end 78.249999 147.810001) (width 0.25) (layer F.Cu) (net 22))
 (segment (start 71.755 146.685) (end 72.880001 147.810001) (width 0.25) (layer F.Cu) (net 22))
 (segment (start 59.055 102.235) (end 63.5 102.235) (width 0.25) (layer F.Cu) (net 23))
 (segment (start 59.055 99.695) (end 63.5 99.695) (width 0.25) (layer F.Cu) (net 24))
 (segment (start 59.055 97.155) (end 63.5 97.155) (width 0.25) (layer F.Cu) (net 25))
 (segment (start 59.055 94.615) (end 63.5 94.615) (width 0.25) (layer F.Cu) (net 26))
 (segment (start 59.055 92.075) (end 63.5 92.075) (width 0.25) (layer F.Cu) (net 27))
 (segment (start 79.865001 93.489999) (end 79.865001 90.660001) (width 0.25) (layer F.Cu) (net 28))
 (segment (start 78.74 94.615) (end 79.865001 93.489999) (width 0.25) (layer F.Cu) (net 28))
 (segment (start 78.74 89.535) (end 59.055 89.535) (width 0.25) (layer F.Cu) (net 28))
 (segment (start 79.865001 90.660001) (end 78.74 89.535) (width 0.25) (layer F.Cu) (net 28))
 (segment (start 76.83641 86.995) (end 59.055 86.995) (width 0.25) (layer F.Cu) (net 29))
 (segment (start 80.31501 90.4736) (end 76.83641 86.995) (width 0.25) (layer F.Cu) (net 29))
 (segment (start 80.31501 95.57999) (end 80.31501 90.4736) (width 0.25) (layer F.Cu) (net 29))
 (segment (start 78.74 97.155) (end 80.31501 95.57999) (width 0.25) (layer F.Cu) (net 29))
 (segment (start 74.93282 84.455) (end 59.055 84.455) (width 0.25) (layer F.Cu) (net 30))
 (segment (start 80.765019 90.287199) (end 74.93282 84.455) (width 0.25) (layer F.Cu) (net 30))
 (segment (start 80.765019 97.669981) (end 80.765019 90.287199) (width 0.25) (layer F.Cu) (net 30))
 (segment (start 78.74 99.695) (end 80.765019 97.669981) (width 0.25) (layer F.Cu) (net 30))
 (via (at 74.295 131.445) (size 0.8) (drill 0.4) (layers F.Cu B.Cu) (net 34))
 (segment (start 64.135 146.685) (end 64.135 141.605) (width 0.25) (layer F.Cu) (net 34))
 (segment (start 64.135 141.605) (end 74.295 131.445) (width 0.25) (layer F.Cu) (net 34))
 (segment (start 74.295 131.445) (end 74.295 96.52) (width 0.25) (layer B.Cu) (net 34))
 (segment (start 74.295 96.52) (end 78.74 92.075) (width 0.25) (layer B.Cu) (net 34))
 (segment (start 64.135 151.765) (end 66.675 154.305) (width 0.25) (layer F.Cu) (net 34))
 (segment (start 64.135 146.685) (end 64.135 151.765) (width 0.25) (layer F.Cu) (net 34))
 (segment (start 66.675 154.305) (end 69.215 154.305) (width 0.25) (layer F.Cu) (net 34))
 (segment (start 73.169999 153.179999) (end 74.295 154.305) (width 0.25) (layer F.Cu) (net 34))
 (segment (start 70.340001 153.179999) (end 73.169999 153.179999) (width 0.25) (layer F.Cu) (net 34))
 (segment (start 69.215 154.305) (end 70.340001 153.179999) (width 0.25) (layer F.Cu) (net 34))
 (segment (start 74.295 154.305) (end 76.835 154.305) (width 0.25) (layer F.Cu) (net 34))
 (segment (start 60.96 74.295) (end 78.74 92.075) (width 0.25) (layer B.Cu) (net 34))
 (segment (start 59.055 74.295) (end 60.96 74.295) (width 0.25) (layer B.Cu) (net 34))
 (segment (start 76.979999 98.569999) (end 81.705001 98.569999) (width 0.25) (layer B.Cu) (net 34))
 (segment (start 84.310001 106.189999) (end 83.185 107.315) (width 0.25) (layer B.Cu) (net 34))
 (segment (start 84.310001 101.174999) (end 84.310001 106.189999) (width 0.25) (layer B.Cu) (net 34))
 (segment (start 81.705001 98.569999) (end 84.310001 101.174999) (width 0.25) (layer B.Cu) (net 34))
 (segment (start 74.93 96.52) (end 76.979999 98.569999) (width 0.25) (layer B.Cu) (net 34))
 (segment (start 74.295 96.52) (end 74.93 96.52) (width 0.25) (layer B.Cu) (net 34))
 (segment (start 82.059999 111.269999) (end 83.185 112.395) (width 0.25) (layer B.Cu) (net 34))
 (segment (start 82.059999 108.440001) (end 82.059999 111.269999) (width 0.25) (layer B.Cu) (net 34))
 (segment (start 83.185 107.315) (end 82.059999 108.440001) (width 0.25) (layer B.Cu) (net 34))
 (segment (start 82.059999 116.349999) (end 83.185 117.475) (width 0.25) (layer B.Cu) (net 34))
 (segment (start 82.059999 113.520001) (end 82.059999 116.349999) (width 0.25) (layer B.Cu) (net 34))
 (segment (start 83.185 112.395) (end 82.059999 113.520001) (width 0.25) (layer B.Cu) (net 34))
 (segment (start 89.679999 108.729999) (end 90.805 109.855) (width 0.25) (layer F.Cu) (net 34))
 (segment (start 89.679999 105.900001) (end 89.679999 108.729999) (width 0.25) (layer F.Cu) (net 34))
 (segment (start 90.805 104.775) (end 89.679999 105.900001) (width 0.25) (layer F.Cu) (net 34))
 (segment (start 89.679999 113.809999) (end 90.805 114.935) (width 0.25) (layer F.Cu) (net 34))
 (segment (start 89.679999 110.980001) (end 89.679999 113.809999) (width 0.25) (layer F.Cu) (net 34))
 (segment (start 90.805 109.855) (end 89.679999 110.980001) (width 0.25) (layer F.Cu) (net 34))
 (segment (start 85.725 114.935) (end 83.185 117.475) (width 0.25) (layer F.Cu) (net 34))
 (segment (start 90.805 114.935) (end 85.725 114.935) (width 0.25) (layer F.Cu) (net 34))
 (segment (start 62.86923 71.755) (end 90.805 99.69077) (width 0.25) (layer F.Cu) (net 35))
 (segment (start 90.805 99.69077) (end 90.805 102.235) (width 0.25) (layer F.Cu) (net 35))
 (segment (start 59.055 71.755) (end 62.86923 71.755) (width 0.25) (layer F.Cu) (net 35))
 (segment (start 63.5 125.095) (end 65.40359 125.095) (width 0.25) (layer B.Cu) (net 35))
 (via (at 65.95 140.97) (size 0.8) (drill 0.4) (layers F.Cu B.Cu) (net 35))
 (segment (start 65.40359 125.095) (end 65.95 125.64141) (width 0.25) (layer B.Cu) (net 35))
 (segment (start 65.95 125.64141) (end 65.95 140.97) (width 0.25) (layer B.Cu) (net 35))
 (segment (start 65.95 140.97) (end 67.31 140.97) (width 0.25) (layer F.Cu) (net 35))
 (via (at 73.025 135.255) (size 0.8) (drill 0.4) (layers F.Cu B.Cu) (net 35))
 (segment (start 67.31 140.97) (end 67.400001 140.879999) (width 0.25) (layer F.Cu) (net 35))
 (segment (start 67.400001 140.879999) (end 73.025 135.255) (width 0.25) (layer F.Cu) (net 35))
 (segment (start 73.025 135.255) (end 75.565 135.255) (width 0.25) (layer B.Cu) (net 35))
 (segment (start 75.565 135.255) (end 75.565 134.62) (width 0.25) (layer B.Cu) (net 35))
 (segment (start 89.679999 103.360001) (end 90.805 102.235) (width 0.25) (layer B.Cu) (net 35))
 (segment (start 89.679999 120.505001) (end 89.679999 103.360001) (width 0.25) (layer B.Cu) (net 35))
 (segment (start 75.565 134.62) (end 89.679999 120.505001) (width 0.25) (layer B.Cu) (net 35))
 (segment (start 80.500001 153.179999) (end 80.500001 140.190001) (width 0.25) (layer B.Cu) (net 35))
 (segment (start 79.375 154.305) (end 80.500001 153.179999) (width 0.25) (layer B.Cu) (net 35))
 (segment (start 80.500001 140.190001) (end 75.565 135.255) (width 0.25) (layer B.Cu) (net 35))
 (segment (start 66.675 125.73) (end 63.5 122.555) (width 0.25) (layer B.Cu) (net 42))
 (segment (start 66.675 146.685) (end 66.675 125.73) (width 0.25) (layer B.Cu) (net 42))
 (segment (start 79.865001 101.694999) (end 79.865001 128.414999) (width 0.25) (layer F.Cu) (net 43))
 (segment (start 79.280001 101.109999) (end 79.865001 101.694999) (width 0.25) (layer F.Cu) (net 43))
 (segment (start 63.5 109.855) (end 72.245001 101.109999) (width 0.25) (layer F.Cu) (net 43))
 (segment (start 72.245001 101.109999) (end 79.280001 101.109999) (width 0.25) (layer F.Cu) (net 43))
 (segment (start 74.295 133.985) (end 74.295 146.685) (width 0.25) (layer F.Cu) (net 43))
 (segment (start 79.865001 128.414999) (end 74.295 133.985) (width 0.25) (layer F.Cu) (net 43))
 (segment (start 83.185 104.775) (end 81.915 103.505) (width 0.25) (layer B.Cu) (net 40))
 (via (at 75.565 103.505) (size 0.8) (drill 0.4) (layers F.Cu B.Cu) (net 40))
 (segment (start 81.915 103.505) (end 75.565 103.505) (width 0.25) (layer B.Cu) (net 40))
 (via (at 71.12 103.505) (size 0.8) (drill 0.4) (layers F.Cu B.Cu) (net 40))
 (segment (start 75.565 103.505) (end 71.12 103.505) (width 0.25) (layer F.Cu) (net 40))
 (segment (start 64.77 103.505) (end 63.5 104.775) (width 0.25) (layer B.Cu) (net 40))
 (segment (start 71.12 103.505) (end 64.77 103.505) (width 0.25) (layer B.Cu) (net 40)))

